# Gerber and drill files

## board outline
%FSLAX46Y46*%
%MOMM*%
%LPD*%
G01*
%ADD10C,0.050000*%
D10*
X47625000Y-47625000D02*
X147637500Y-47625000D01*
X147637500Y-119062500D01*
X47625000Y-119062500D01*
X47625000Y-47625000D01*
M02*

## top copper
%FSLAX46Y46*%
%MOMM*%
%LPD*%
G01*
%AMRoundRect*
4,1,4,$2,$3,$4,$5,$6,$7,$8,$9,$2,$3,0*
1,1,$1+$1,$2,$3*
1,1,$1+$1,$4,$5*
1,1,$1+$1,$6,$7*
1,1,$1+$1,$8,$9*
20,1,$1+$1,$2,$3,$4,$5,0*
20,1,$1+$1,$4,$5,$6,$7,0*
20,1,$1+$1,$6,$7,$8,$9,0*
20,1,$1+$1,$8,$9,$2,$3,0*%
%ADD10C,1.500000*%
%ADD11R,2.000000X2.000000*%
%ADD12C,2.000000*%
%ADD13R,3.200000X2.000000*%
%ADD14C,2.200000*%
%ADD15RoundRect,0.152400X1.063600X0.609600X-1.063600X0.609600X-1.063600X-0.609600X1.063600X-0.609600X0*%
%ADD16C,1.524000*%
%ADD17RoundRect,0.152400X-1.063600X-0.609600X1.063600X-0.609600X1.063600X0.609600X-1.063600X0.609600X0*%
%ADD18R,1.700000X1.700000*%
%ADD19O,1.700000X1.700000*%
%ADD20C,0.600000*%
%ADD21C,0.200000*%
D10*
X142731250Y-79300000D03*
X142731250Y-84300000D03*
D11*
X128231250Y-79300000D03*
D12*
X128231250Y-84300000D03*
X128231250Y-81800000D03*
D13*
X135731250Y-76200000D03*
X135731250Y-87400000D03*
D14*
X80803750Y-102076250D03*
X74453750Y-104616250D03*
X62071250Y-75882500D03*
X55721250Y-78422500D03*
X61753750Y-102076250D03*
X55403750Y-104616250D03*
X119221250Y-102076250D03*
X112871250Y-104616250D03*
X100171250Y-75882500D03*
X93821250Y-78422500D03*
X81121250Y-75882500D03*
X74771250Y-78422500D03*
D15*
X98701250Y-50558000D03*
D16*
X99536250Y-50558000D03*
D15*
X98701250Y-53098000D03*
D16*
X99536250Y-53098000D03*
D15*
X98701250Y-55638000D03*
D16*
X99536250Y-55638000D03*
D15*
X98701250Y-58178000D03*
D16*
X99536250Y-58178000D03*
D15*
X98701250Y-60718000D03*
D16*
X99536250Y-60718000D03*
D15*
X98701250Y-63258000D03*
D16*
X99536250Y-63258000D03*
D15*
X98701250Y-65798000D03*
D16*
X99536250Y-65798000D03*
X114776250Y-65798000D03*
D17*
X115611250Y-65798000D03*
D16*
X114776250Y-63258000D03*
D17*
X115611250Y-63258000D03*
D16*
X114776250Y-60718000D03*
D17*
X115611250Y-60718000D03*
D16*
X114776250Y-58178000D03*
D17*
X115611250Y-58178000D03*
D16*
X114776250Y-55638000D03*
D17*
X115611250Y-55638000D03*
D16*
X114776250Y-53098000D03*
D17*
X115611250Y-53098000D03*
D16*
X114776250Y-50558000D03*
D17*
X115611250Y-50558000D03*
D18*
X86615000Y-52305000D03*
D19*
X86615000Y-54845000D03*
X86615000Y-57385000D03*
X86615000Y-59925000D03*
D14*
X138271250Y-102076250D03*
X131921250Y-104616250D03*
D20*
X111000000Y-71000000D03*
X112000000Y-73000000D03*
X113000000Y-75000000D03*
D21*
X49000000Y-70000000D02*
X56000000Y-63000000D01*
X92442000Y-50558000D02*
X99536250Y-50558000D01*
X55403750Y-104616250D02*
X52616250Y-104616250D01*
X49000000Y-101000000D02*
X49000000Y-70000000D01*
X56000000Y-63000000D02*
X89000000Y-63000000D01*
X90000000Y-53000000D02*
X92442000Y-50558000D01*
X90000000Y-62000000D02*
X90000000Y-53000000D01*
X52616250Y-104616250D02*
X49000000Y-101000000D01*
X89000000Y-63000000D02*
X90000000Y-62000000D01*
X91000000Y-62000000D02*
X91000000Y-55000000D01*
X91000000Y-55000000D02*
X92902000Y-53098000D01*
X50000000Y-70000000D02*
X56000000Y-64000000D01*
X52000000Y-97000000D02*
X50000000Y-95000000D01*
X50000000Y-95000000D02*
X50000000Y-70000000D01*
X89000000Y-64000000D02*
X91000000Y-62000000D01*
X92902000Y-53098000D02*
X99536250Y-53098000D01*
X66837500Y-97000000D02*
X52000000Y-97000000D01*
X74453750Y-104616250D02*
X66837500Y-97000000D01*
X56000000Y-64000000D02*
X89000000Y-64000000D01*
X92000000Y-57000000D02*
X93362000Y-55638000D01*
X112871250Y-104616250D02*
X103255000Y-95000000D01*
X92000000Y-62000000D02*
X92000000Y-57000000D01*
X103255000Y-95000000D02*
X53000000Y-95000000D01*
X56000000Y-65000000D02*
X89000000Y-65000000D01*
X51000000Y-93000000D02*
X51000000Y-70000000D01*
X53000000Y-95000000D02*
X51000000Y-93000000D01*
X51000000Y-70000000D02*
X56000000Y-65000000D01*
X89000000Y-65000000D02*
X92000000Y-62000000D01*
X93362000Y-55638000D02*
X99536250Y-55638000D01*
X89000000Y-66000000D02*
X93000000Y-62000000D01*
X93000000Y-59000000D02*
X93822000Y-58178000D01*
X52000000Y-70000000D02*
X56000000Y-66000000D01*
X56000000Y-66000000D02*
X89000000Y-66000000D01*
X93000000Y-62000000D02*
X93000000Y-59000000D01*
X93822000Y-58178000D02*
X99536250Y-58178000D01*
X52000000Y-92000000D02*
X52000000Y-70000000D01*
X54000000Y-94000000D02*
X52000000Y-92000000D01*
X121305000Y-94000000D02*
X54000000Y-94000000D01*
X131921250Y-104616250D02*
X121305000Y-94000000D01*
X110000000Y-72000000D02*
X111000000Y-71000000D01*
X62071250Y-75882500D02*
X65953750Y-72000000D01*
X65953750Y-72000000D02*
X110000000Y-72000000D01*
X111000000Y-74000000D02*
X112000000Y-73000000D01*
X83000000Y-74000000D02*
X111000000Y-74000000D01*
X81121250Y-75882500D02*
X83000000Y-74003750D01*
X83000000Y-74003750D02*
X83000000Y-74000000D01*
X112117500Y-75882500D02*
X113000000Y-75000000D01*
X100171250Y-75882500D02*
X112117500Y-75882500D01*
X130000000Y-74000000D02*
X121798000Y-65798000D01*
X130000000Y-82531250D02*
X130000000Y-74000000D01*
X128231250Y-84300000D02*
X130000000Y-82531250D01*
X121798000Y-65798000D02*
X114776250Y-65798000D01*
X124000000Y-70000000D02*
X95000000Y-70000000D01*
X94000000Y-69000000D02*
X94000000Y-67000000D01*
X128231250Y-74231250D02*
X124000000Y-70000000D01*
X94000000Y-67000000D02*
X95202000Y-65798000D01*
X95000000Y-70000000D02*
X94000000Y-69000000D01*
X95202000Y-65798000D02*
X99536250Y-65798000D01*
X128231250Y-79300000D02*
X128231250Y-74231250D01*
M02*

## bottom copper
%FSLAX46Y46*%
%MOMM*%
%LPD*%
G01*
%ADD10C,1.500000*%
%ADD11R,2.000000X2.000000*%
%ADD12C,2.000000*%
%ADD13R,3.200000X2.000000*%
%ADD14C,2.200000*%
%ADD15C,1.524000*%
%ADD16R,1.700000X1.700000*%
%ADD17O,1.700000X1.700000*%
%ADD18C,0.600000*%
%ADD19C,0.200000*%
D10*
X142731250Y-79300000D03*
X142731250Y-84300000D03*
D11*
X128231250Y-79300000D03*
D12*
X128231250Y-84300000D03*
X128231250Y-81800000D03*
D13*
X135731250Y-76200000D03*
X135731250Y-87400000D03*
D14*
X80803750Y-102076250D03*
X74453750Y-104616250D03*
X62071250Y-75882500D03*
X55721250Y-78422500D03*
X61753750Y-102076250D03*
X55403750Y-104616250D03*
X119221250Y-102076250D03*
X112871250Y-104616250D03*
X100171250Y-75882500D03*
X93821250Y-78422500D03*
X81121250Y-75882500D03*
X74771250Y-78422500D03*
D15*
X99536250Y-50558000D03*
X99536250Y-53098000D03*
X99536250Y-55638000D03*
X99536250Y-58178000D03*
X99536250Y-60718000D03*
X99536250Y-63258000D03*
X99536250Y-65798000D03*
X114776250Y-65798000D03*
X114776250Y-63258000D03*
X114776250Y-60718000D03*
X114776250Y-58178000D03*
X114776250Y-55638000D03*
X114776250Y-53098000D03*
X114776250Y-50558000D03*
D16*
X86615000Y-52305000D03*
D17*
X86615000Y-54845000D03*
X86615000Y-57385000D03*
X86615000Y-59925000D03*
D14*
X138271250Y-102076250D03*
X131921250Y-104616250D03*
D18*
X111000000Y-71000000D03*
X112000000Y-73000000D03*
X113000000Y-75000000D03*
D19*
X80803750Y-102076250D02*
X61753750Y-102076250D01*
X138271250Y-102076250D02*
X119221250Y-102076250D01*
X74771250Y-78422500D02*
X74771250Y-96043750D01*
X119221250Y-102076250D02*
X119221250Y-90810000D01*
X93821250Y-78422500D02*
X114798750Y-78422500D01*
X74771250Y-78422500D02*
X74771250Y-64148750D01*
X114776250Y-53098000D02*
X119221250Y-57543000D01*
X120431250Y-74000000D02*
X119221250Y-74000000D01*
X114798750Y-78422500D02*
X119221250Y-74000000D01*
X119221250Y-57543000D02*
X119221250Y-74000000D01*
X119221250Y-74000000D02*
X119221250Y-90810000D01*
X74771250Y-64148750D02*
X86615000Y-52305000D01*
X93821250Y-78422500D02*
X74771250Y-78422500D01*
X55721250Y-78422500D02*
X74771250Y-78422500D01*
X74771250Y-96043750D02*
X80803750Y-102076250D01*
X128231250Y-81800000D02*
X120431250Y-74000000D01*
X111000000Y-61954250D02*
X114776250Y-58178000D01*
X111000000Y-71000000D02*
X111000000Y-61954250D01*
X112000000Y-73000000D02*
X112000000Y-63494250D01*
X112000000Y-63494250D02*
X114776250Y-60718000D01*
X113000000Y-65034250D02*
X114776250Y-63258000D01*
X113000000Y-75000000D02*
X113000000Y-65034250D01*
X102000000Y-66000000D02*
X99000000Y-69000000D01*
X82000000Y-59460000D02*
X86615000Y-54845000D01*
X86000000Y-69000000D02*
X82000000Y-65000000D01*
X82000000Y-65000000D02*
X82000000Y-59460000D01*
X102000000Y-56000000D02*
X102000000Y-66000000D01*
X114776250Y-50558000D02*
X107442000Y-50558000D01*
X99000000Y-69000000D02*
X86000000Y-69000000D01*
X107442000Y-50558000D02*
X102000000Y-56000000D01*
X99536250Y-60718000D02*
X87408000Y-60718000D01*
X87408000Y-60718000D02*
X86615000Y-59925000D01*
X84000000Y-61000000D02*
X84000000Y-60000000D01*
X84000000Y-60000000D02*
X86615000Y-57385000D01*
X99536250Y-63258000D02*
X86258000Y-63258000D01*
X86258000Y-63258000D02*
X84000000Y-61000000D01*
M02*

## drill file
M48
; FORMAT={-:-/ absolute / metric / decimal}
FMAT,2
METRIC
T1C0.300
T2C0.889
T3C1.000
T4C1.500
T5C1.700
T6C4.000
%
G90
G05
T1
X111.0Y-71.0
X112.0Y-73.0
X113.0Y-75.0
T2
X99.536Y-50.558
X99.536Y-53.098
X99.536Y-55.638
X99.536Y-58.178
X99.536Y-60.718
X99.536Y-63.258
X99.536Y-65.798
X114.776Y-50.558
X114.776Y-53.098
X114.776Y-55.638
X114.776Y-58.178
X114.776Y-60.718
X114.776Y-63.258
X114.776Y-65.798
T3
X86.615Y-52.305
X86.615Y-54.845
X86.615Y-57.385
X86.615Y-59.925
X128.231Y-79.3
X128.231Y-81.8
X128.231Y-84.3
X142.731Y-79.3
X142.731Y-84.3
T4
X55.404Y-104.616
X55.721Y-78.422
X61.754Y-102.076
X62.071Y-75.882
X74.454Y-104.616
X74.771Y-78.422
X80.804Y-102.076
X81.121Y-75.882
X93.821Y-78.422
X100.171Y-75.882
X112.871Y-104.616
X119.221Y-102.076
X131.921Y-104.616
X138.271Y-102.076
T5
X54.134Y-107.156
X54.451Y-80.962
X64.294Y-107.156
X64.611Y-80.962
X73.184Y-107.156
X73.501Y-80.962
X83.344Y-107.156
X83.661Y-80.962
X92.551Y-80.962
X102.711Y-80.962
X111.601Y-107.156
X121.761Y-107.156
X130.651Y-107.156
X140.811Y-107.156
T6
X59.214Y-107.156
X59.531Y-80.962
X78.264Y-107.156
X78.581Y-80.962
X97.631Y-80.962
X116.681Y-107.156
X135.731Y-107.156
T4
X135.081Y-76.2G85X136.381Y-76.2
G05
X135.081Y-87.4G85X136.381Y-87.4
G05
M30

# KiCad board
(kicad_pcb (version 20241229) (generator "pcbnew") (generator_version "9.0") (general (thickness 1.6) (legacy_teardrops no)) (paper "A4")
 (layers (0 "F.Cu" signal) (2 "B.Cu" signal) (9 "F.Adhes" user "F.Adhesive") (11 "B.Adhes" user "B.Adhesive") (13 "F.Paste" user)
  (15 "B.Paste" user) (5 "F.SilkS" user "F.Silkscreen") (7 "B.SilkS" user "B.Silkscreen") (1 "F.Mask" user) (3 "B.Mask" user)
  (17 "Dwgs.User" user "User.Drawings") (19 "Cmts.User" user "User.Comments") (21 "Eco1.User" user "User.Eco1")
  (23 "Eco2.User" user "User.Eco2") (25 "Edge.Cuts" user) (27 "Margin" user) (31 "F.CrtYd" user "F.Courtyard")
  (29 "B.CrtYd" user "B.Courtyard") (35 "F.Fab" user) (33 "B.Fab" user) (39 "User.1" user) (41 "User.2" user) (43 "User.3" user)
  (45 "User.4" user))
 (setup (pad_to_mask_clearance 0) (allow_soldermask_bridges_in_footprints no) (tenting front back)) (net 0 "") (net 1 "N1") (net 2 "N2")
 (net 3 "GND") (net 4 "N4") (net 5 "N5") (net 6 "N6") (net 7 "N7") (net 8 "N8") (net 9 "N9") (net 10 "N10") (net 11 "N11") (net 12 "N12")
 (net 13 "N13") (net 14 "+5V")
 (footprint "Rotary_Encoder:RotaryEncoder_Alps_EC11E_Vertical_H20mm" (layer "F.Cu") (at 128.23125 79.3)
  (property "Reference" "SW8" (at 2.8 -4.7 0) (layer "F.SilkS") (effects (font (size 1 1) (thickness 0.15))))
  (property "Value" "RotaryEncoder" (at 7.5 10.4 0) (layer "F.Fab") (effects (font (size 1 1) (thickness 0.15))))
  (pad "" thru_hole circle (at 14.5 0) (size 1.5 1.5) (drill 1) (layers "*.Cu" "*.Mask") (remove_unused_layers no))
  (pad "" thru_hole circle (at 14.5 5) (size 1.5 1.5) (drill 1) (layers "*.Cu" "*.Mask") (remove_unused_layers no))
  (pad "A" thru_hole rect (at 0 0) (size 2 2) (drill 1) (layers "*.Cu" "*.Mask") (remove_unused_layers no) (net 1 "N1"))
  (pad "B" thru_hole circle (at 0 5) (size 2 2) (drill 1) (layers "*.Cu" "*.Mask") (remove_unused_layers no) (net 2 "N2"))
  (pad "C" thru_hole circle (at 0 2.5) (size 2 2) (drill 1) (layers "*.Cu" "*.Mask") (remove_unused_layers no) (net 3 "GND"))
  (pad "MP" thru_hole rect (at 7.5 -3.1) (size 3.2 2) (drill oval 2.8 1.5) (layers "*.Cu" "*.Mask") (remove_unused_layers no))
  (pad "MP" thru_hole rect (at 7.5 8.1) (size 3.2 2) (drill oval 2.8 1.5) (layers "*.Cu" "*.Mask") (remove_unused_layers no)))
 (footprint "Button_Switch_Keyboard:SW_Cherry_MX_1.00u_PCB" (layer "F.Cu") (at 80.80375 102.07625)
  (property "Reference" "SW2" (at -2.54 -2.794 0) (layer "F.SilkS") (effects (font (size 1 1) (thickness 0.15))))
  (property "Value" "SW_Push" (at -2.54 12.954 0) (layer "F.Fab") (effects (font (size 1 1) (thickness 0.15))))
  (pad "" np_thru_hole circle (at -7.62 5.08) (size 1.7 1.7) (drill 1.7) (layers "*.Cu" "*.Mask"))
  (pad "" np_thru_hole circle (at -2.54 5.08) (size 4 4) (drill 4) (layers "*.Cu" "*.Mask"))
  (pad "" np_thru_hole circle (at 2.54 5.08) (size 1.7 1.7) (drill 1.7) (layers "*.Cu" "*.Mask"))
  (pad "1" thru_hole circle (at 0 0) (size 2.2 2.2) (drill 1.5) (layers "*.Cu" "*.Mask") (remove_unused_layers no) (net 3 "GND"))
  (pad "2" thru_hole circle (at -6.35 2.54) (size 2.2 2.2) (drill 1.5) (layers "*.Cu" "*.Mask") (remove_unused_layers no) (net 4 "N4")))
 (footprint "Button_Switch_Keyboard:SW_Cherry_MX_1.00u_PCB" (layer "F.Cu") (at 62.07125 75.8825)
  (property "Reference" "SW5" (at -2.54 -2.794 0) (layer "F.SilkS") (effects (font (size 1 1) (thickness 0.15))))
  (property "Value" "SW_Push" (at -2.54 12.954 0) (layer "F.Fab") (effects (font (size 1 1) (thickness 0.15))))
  (pad "" np_thru_hole circle (at -7.62 5.08) (size 1.7 1.7) (drill 1.7) (layers "*.Cu" "*.Mask"))
  (pad "" np_thru_hole circle (at -2.54 5.08) (size 4 4) (drill 4) (layers "*.Cu" "*.Mask"))
  (pad "" np_thru_hole circle (at 2.54 5.08) (size 1.7 1.7) (drill 1.7) (layers "*.Cu" "*.Mask"))
  (pad "1" thru_hole circle (at 0 0) (size 2.2 2.2) (drill 1.5) (layers "*.Cu" "*.Mask") (remove_unused_layers no) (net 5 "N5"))
  (pad "2" thru_hole circle (at -6.35 2.54) (size 2.2 2.2) (drill 1.5) (layers "*.Cu" "*.Mask") (remove_unused_layers no) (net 3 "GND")))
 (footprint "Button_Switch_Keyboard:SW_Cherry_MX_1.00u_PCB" (layer "F.Cu") (at 61.75375 102.07625)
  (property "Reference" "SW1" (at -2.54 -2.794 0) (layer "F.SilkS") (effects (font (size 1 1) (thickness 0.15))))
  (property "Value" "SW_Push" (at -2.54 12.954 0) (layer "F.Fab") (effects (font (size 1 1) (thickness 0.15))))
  (pad "" np_thru_hole circle (at -7.62 5.08) (size 1.7 1.7) (drill 1.7) (layers "*.Cu" "*.Mask"))
  (pad "" np_thru_hole circle (at -2.54 5.08) (size 4 4) (drill 4) (layers "*.Cu" "*.Mask"))
  (pad "" np_thru_hole circle (at 2.54 5.08) (size 1.7 1.7) (drill 1.7) (layers "*.Cu" "*.Mask"))
  (pad "1" thru_hole circle (at 0 0) (size 2.2 2.2) (drill 1.5) (layers "*.Cu" "*.Mask") (remove_unused_layers no) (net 3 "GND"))
  (pad "2" thru_hole circle (at -6.35 2.54) (size 2.2 2.2) (drill 1.5) (layers "*.Cu" "*.Mask") (remove_unused_layers no) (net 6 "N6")))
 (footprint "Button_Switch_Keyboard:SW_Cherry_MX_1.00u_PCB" (layer "F.Cu") (at 119.22125 102.07625)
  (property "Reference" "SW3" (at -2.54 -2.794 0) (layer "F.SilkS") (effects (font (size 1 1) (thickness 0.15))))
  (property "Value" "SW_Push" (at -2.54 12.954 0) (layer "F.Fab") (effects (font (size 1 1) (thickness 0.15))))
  (pad "" np_thru_hole circle (at -7.62 5.08) (size 1.7 1.7) (drill 1.7) (layers "*.Cu" "*.Mask"))
  (pad "" np_thru_hole circle (at -2.54 5.08) (size 4 4) (drill 4) (layers "*.Cu" "*.Mask"))
  (pad "" np_thru_hole circle (at 2.54 5.08) (size 1.7 1.7) (drill 1.7) (layers "*.Cu" "*.Mask"))
  (pad "1" thru_hole circle (at 0 0) (size 2.2 2.2) (drill 1.5) (layers "*.Cu" "*.Mask") (remove_unused_layers no) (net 3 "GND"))
  (pad "2" thru_hole circle (at -6.35 2.54) (size 2.2 2.2) (drill 1.5) (layers "*.Cu" "*.Mask") (remove_unused_layers no) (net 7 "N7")))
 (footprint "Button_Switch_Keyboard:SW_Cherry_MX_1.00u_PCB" (layer "F.Cu") (at 100.17125 75.8825)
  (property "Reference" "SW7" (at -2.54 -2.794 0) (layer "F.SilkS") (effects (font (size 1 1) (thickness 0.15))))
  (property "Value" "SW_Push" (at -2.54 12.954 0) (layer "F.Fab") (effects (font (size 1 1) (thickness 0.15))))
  (pad "" np_thru_hole circle (at -7.62 5.08) (size 1.7 1.7) (drill 1.7) (layers "*.Cu" "*.Mask"))
  (pad "" np_thru_hole circle (at -2.54 5.08) (size 4 4) (drill 4) (layers "*.Cu" "*.Mask"))
  (pad "" np_thru_hole circle (at 2.54 5.08) (size 1.7 1.7) (drill 1.7) (layers "*.Cu" "*.Mask"))
  (pad "1" thru_hole circle (at 0 0) (size 2.2 2.2) (drill 1.5) (layers "*.Cu" "*.Mask") (remove_unused_layers no) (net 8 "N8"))
  (pad "2" thru_hole circle (at -6.35 2.54) (size 2.2 2.2) (drill 1.5) (layers "*.Cu" "*.Mask") (remove_unused_layers no) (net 3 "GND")))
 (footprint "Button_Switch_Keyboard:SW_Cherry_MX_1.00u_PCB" (layer "F.Cu") (at 81.12125 75.8825)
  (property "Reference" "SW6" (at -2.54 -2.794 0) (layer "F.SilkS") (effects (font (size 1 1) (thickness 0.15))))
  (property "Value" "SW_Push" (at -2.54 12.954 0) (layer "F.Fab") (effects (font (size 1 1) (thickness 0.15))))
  (pad "" np_thru_hole circle (at -7.62 5.08) (size 1.7 1.7) (drill 1.7) (layers "*.Cu" "*.Mask"))
  (pad "" np_thru_hole circle (at -2.54 5.08) (size 4 4) (drill 4) (layers "*.Cu" "*.Mask"))
  (pad "" np_thru_hole circle (at 2.54 5.08) (size 1.7 1.7) (drill 1.7) (layers "*.Cu" "*.Mask"))
  (pad "1" thru_hole circle (at 0 0) (size 2.2 2.2) (drill 1.5) (layers "*.Cu" "*.Mask") (remove_unused_layers no) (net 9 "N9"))
  (pad "2" thru_hole circle (at -6.35 2.54) (size 2.2 2.2) (drill 1.5) (layers "*.Cu" "*.Mask") (remove_unused_layers no) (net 3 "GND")))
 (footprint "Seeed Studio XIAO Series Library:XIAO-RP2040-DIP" (layer "F.Cu") (at 107.15625 58.178)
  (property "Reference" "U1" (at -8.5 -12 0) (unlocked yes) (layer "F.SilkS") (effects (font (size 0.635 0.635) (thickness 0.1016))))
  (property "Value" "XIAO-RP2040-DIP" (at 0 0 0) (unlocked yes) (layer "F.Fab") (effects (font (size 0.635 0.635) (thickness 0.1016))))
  (pad "1" smd roundrect (at -8.455 -7.62 180) (size 2.432 1.524) (layers "F.Cu" "F.Mask") (roundrect_rratio 0.1) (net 6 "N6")
   (thermal_bridge_angle 45))
  (pad "1" thru_hole circle (at -7.62 -7.62 180) (size 1.524 1.524) (drill 0.889) (layers "*.Cu" "*.Mask") (remove_unused_layers no)
   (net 6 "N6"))
  (pad "2" smd roundrect (at -8.455 -5.08 180) (size 2.432 1.524) (layers "F.Cu" "F.Mask") (roundrect_rratio 0.1) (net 4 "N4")
   (thermal_bridge_angle 45))
  (pad "2" thru_hole circle (at -7.62 -5.08 180) (size 1.524 1.524) (drill 0.889) (layers "*.Cu" "*.Mask") (remove_unused_layers no)
   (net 4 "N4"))
  (pad "3" smd roundrect (at -8.455 -2.54 180) (size 2.432 1.524) (layers "F.Cu" "F.Mask") (roundrect_rratio 0.1) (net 7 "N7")
   (thermal_bridge_angle 45))
  (pad "3" thru_hole circle (at -7.62 -2.54 180) (size 1.524 1.524) (drill 0.889) (layers "*.Cu" "*.Mask") (remove_unused_layers no)
   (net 7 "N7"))
  (pad "4" smd roundrect (at -8.455 0 180) (size 2.432 1.524) (layers "F.Cu" "F.Mask") (roundrect_rratio 0.1) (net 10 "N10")
   (thermal_bridge_angle 45))
  (pad "4" thru_hole circle (at -7.62 0 180) (size 1.524 1.524) (drill 0.889) (layers "*.Cu" "*.Mask") (remove_unused_layers no)
   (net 10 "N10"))
  (pad "5" smd roundrect (at -8.455 2.54 180) (size 2.432 1.524) (layers "F.Cu" "F.Mask") (roundrect_rratio 0.1) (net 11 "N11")
   (thermal_bridge_angle 45))
  (pad "5" thru_hole circle (at -7.62 2.54 180) (size 1.524 1.524) (drill 0.889) (layers "*.Cu" "*.Mask") (remove_unused_layers no)
   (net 11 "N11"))
  (pad "6" smd roundrect (at -8.455 5.08 180) (size 2.432 1.524) (layers "F.Cu" "F.Mask") (roundrect_rratio 0.1) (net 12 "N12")
   (thermal_bridge_angle 45))
  (pad "6" thru_hole circle (at -7.62 5.08 180) (size 1.524 1.524) (drill 0.889) (layers "*.Cu" "*.Mask") (remove_unused_layers no)
   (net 12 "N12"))
  (pad "7" smd roundrect (at -8.455 7.62 180) (size 2.432 1.524) (layers "F.Cu" "F.Mask") (roundrect_rratio 0.1) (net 1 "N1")
   (thermal_bridge_angle 45))
  (pad "7" thru_hole circle (at -7.62 7.62 180) (size 1.524 1.524) (drill 0.889) (layers "*.Cu" "*.Mask") (remove_unused_layers no)
   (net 1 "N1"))
  (pad "8" thru_hole circle (at 7.62 7.62) (size 1.524 1.524) (drill 0.889) (layers "*.Cu" "*.Mask") (remove_unused_layers no) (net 2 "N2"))
  (pad "8" smd roundrect (at 8.455 7.62) (size 2.432 1.524) (layers "F.Cu" "F.Mask") (roundrect_rratio 0.1) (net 2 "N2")
   (thermal_bridge_angle 45))
  (pad "9" thru_hole circle (at 7.62 5.08) (size 1.524 1.524) (drill 0.889) (layers "*.Cu" "*.Mask") (remove_unused_layers no) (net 8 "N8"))
  (pad "9" smd roundrect (at 8.455 5.08) (size 2.432 1.524) (layers "F.Cu" "F.Mask") (roundrect_rratio 0.1) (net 8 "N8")
   (thermal_bridge_angle 45))
  (pad "10" thru_hole circle (at 7.62 2.54) (size 1.524 1.524) (drill 0.889) (layers "*.Cu" "*.Mask") (remove_unused_layers no) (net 9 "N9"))
  (pad "10" smd roundrect (at 8.455 2.54) (size 2.432 1.524) (layers "F.Cu" "F.Mask") (roundrect_rratio 0.1) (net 9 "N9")
   (thermal_bridge_angle 45))
  (pad "11" thru_hole circle (at 7.62 0) (size 1.524 1.524) (drill 0.889) (layers "*.Cu" "*.Mask") (remove_unused_layers no) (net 5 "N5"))
  (pad "11" smd roundrect (at 8.455 0) (size 2.432 1.524) (layers "F.Cu" "F.Mask") (roundrect_rratio 0.1) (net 5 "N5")
   (thermal_bridge_angle 45))
  (pad "12" thru_hole circle (at 7.62 -2.54) (size 1.524 1.524) (drill 0.889) (layers "*.Cu" "*.Mask") (remove_unused_layers no)
   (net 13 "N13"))
  (pad "12" smd roundrect (at 8.455 -2.54) (size 2.432 1.524) (layers "F.Cu" "F.Mask") (roundrect_rratio 0.1) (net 13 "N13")
   (thermal_bridge_angle 45))
  (pad "13" thru_hole circle (at 7.62 -5.08) (size 1.524 1.524) (drill 0.889) (layers "*.Cu" "*.Mask") (remove_unused_layers no)
   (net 3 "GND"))
  (pad "13" smd roundrect (at 8.455 -5.08) (size 2.432 1.524) (layers "F.Cu" "F.Mask") (roundrect_rratio 0.1) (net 3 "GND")
   (thermal_bridge_angle 45))
  (pad "14" thru_hole circle (at 7.62 -7.62) (size 1.524 1.524) (drill 0.889) (layers "*.Cu" "*.Mask") (remove_unused_layers no)
   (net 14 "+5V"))
  (pad "14" smd roundrect (at 8.455 -7.62) (size 2.432 1.524) (layers "F.Cu" "F.Mask") (roundrect_rratio 0.1) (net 14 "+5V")
   (thermal_bridge_angle 45)))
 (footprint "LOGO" (layer "F.Cu") (at 134 58)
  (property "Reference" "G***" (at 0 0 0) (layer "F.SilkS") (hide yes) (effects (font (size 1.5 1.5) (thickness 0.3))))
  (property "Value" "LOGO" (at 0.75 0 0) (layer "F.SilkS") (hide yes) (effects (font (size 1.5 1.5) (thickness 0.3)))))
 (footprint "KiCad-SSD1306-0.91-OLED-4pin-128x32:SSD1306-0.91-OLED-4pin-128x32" (layer "F.Cu") (at 50.115 50.115)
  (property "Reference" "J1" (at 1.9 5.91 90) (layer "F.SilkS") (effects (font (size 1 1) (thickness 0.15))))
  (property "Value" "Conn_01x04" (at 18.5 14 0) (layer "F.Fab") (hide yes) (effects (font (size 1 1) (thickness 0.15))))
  (pad "1" thru_hole rect (at 36.5 2.19) (size 1.7 1.7) (drill 1) (layers "*.Cu" "*.Mask") (remove_unused_layers no) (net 3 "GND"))
  (pad "2" thru_hole oval (at 36.5 4.73) (size 1.7 1.7) (drill 1) (layers "*.Cu" "*.Mask") (remove_unused_layers no) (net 14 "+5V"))
  (pad "3" thru_hole oval (at 36.5 7.27) (size 1.7 1.7) (drill 1) (layers "*.Cu" "*.Mask") (remove_unused_layers no) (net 12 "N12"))
  (pad "4" thru_hole oval (at 36.5 9.81) (size 1.7 1.7) (drill 1) (layers "*.Cu" "*.Mask") (remove_unused_layers no) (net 11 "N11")))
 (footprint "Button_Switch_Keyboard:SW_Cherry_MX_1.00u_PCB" (layer "F.Cu") (at 138.27125 102.07625)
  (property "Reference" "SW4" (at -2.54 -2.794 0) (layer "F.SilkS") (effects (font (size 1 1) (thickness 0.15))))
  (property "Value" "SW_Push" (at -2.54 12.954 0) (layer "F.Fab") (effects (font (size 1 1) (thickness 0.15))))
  (pad "" np_thru_hole circle (at -7.62 5.08) (size 1.7 1.7) (drill 1.7) (layers "*.Cu" "*.Mask"))
  (pad "" np_thru_hole circle (at -2.54 5.08) (size 4 4) (drill 4) (layers "*.Cu" "*.Mask"))
  (pad "" np_thru_hole circle (at 2.54 5.08) (size 1.7 1.7) (drill 1.7) (layers "*.Cu" "*.Mask"))
  (pad "1" thru_hole circle (at 0 0) (size 2.2 2.2) (drill 1.5) (layers "*.Cu" "*.Mask") (remove_unused_layers no) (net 3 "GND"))
  (pad "2" thru_hole circle (at -6.35 2.54) (size 2.2 2.2) (drill 1.5) (layers "*.Cu" "*.Mask") (remove_unused_layers no) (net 10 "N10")))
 (gr_rect (start 47.625 47.625) (end 147.6375 119.0625) (stroke (width 0.05) (type default)) (fill no) (layer "Edge.Cuts"))
 (segment (start 49 70) (end 56 63) (width 0.2) (layer "F.Cu") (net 6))
 (segment (start 92.442 50.558) (end 99.53625 50.558) (width 0.2) (layer "F.Cu") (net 6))
 (segment (start 55.40375 104.61625) (end 52.61625 104.61625) (width 0.2) (layer "F.Cu") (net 6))
 (segment (start 49 101) (end 49 70) (width 0.2) (layer "F.Cu") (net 6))
 (segment (start 56 63) (end 89 63) (width 0.2) (layer "F.Cu") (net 6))
 (segment (start 90 53) (end 92.442 50.558) (width 0.2) (layer "F.Cu") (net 6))
 (segment (start 90 62) (end 90 53) (width 0.2) (layer "F.Cu") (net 6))
 (segment (start 52.61625 104.61625) (end 49 101) (width 0.2) (layer "F.Cu") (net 6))
 (segment (start 89 63) (end 90 62) (width 0.2) (layer "F.Cu") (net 6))
 (segment (start 80.80375 102.07625) (end 61.75375 102.07625) (width 0.2) (layer "B.Cu") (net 3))
 (segment (start 138.27125 102.07625) (end 119.22125 102.07625) (width 0.2) (layer "B.Cu") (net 3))
 (segment (start 74.77125 78.4225) (end 74.77125 96.04375) (width 0.2) (layer "B.Cu") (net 3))
 (segment (start 119.22125 102.07625) (end 119.22125 90.81) (width 0.2) (layer "B.Cu") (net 3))
 (segment (start 93.82125 78.4225) (end 114.79875 78.4225) (width 0.2) (layer "B.Cu") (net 3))
 (segment (start 74.77125 78.4225) (end 74.77125 64.14875) (width 0.2) (layer "B.Cu") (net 3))
 (segment (start 114.77625 53.098) (end 119.22125 57.543) (width 0.2) (layer "B.Cu") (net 3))
 (segment (start 120.43125 74) (end 119.22125 74) (width 0.2) (layer "B.Cu") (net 3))
 (segment (start 114.79875 78.4225) (end 119.22125 74) (width 0.2) (layer "B.Cu") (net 3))
 (segment (start 119.22125 57.543) (end 119.22125 74) (width 0.2) (layer "B.Cu") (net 3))
 (segment (start 119.22125 74) (end 119.22125 90.81) (width 0.2) (layer "B.Cu") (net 3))
 (segment (start 74.77125 64.14875) (end 86.615 52.305) (width 0.2) (layer "B.Cu") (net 3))
 (segment (start 93.82125 78.4225) (end 74.77125 78.4225) (width 0.2) (layer "B.Cu") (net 3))
 (segment (start 55.72125 78.4225) (end 74.77125 78.4225) (width 0.2) (layer "B.Cu") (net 3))
 (segment (start 74.77125 96.04375) (end 80.80375 102.07625) (width 0.2) (layer "B.Cu") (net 3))
 (segment (start 128.23125 81.8) (end 120.43125 74) (width 0.2) (layer "B.Cu") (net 3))
 (segment (start 91 62) (end 91 55) (width 0.2) (layer "F.Cu") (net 4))
 (segment (start 91 55) (end 92.902 53.098) (width 0.2) (layer "F.Cu") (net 4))
 (segment (start 50 70) (end 56 64) (width 0.2) (layer "F.Cu") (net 4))
 (segment (start 52 97) (end 50 95) (width 0.2) (layer "F.Cu") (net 4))
 (segment (start 50 95) (end 50 70) (width 0.2) (layer "F.Cu") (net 4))
 (segment (start 89 64) (end 91 62) (width 0.2) (layer "F.Cu") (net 4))
 (segment (start 92.902 53.098) (end 99.53625 53.098) (width 0.2) (layer "F.Cu") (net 4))
 (segment (start 66.8375 97) (end 52 97) (width 0.2) (layer "F.Cu") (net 4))
 (segment (start 74.45375 104.61625) (end 66.8375 97) (width 0.2) (layer "F.Cu") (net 4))
 (segment (start 56 64) (end 89 64) (width 0.2) (layer "F.Cu") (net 4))
 (segment (start 92 57) (end 93.362 55.638) (width 0.2) (layer "F.Cu") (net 7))
 (segment (start 112.87125 104.61625) (end 103.255 95) (width 0.2) (layer "F.Cu") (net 7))
 (segment (start 92 62) (end 92 57) (width 0.2) (layer "F.Cu") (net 7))
 (segment (start 103.255 95) (end 53 95) (width 0.2) (layer "F.Cu") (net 7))
 (segment (start 56 65) (end 89 65) (width 0.2) (layer "F.Cu") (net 7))
 (segment (start 51 93) (end 51 70) (width 0.2) (layer "F.Cu") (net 7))
 (segment (start 53 95) (end 51 93) (width 0.2) (layer "F.Cu") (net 7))
 (segment (start 51 70) (end 56 65) (width 0.2) (layer "F.Cu") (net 7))
 (segment (start 89 65) (end 92 62) (width 0.2) (layer "F.Cu") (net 7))
 (segment (start 93.362 55.638) (end 99.53625 55.638) (width 0.2) (layer "F.Cu") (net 7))
 (segment (start 89 66) (end 93 62) (width 0.2) (layer "F.Cu") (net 10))
 (segment (start 93 59) (end 93.822 58.178) (width 0.2) (layer "F.Cu") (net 10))
 (segment (start 52 70) (end 56 66) (width 0.2) (layer "F.Cu") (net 10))
 (segment (start 56 66) (end 89 66) (width 0.2) (layer "F.Cu") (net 10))
 (segment (start 93 62) (end 93 59) (width 0.2) (layer "F.Cu") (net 10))
 (segment (start 93.822 58.178) (end 99.53625 58.178) (width 0.2) (layer "F.Cu") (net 10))
 (segment (start 52 92) (end 52 70) (width 0.2) (layer "F.Cu") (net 10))
 (segment (start 54 94) (end 52 92) (width 0.2) (layer "F.Cu") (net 10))
 (segment (start 121.305 94) (end 54 94) (width 0.2) (layer "F.Cu") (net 10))
 (segment (start 131.92125 104.61625) (end 121.305 94) (width 0.2) (layer "F.Cu") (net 10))
 (segment (start 110 72) (end 111 71) (width 0.2) (layer "F.Cu") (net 5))
 (segment (start 62.07125 75.8825) (end 65.95375 72) (width 0.2) (layer "F.Cu") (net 5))
 (segment (start 65.95375 72) (end 110 72) (width 0.2) (layer "F.Cu") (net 5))
 (via (at 111 71) (size 0.6) (drill 0.3) (layers "F.Cu" "B.Cu") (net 5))
 (segment (start 111 61.95425) (end 114.77625 58.178) (width 0.2) (layer "B.Cu") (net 5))
 (segment (start 111 71) (end 111 61.95425) (width 0.2) (layer "B.Cu") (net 5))
 (segment (start 111 74) (end 112 73) (width 0.2) (layer "F.Cu") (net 9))
 (segment (start 83 74) (end 111 74) (width 0.2) (layer "F.Cu") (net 9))
 (segment (start 81.12125 75.8825) (end 83 74.00375) (width 0.2) (layer "F.Cu") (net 9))
 (segment (start 83 74.00375) (end 83 74) (width 0.2) (layer "F.Cu") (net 9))
 (via (at 112 73) (size 0.6) (drill 0.3) (layers "F.Cu" "B.Cu") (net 9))
 (segment (start 112 73) (end 112 63.49425) (width 0.2) (layer "B.Cu") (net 9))
 (segment (start 112 63.49425) (end 114.77625 60.718) (width 0.2) (layer "B.Cu") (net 9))
 (segment (start 112.1175 75.8825) (end 113 75) (width 0.2) (layer "F.Cu") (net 8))
 (segment (start 100.17125 75.8825) (end 112.1175 75.8825) (width 0.2) (layer "F.Cu") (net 8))
 (via (at 113 75) (size 0.6) (drill 0.3) (layers "F.Cu" "B.Cu") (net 8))
 (segment (start 113 65.03425) (end 114.77625 63.258) (width 0.2) (layer "B.Cu") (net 8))
 (segment (start 113 75) (end 113 65.03425) (width 0.2) (layer "B.Cu") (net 8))
 (segment (start 130 74) (end 121.798 65.798) (width 0.2) (layer "F.Cu") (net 2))
 (segment (start 130 82.53125) (end 130 74) (width 0.2) (layer "F.Cu") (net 2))
 (segment (start 128.23125 84.3) (end 130 82.53125) (width 0.2) (layer "F.Cu") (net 2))
 (segment (start 121.798 65.798) (end 114.77625 65.798) (width 0.2) (layer "F.Cu") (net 2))
 (segment (start 124 70) (end 95 70) (width 0.2) (layer "F.Cu") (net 1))
 (segment (start 94 69) (end 94 67) (width 0.2) (layer "F.Cu") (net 1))
 (segment (start 128.23125 74.23125) (end 124 70) (width 0.2) (layer "F.Cu") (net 1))
 (segment (start 94 67) (end 95.202 65.798) (width 0.2) (layer "F.Cu") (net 1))
 (segment (start 95 70) (end 94 69) (width 0.2) (layer "F.Cu") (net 1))
 (segment (start 95.202 65.798) (end 99.53625 65.798) (width 0.2) (layer "F.Cu") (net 1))
 (segment (start 128.23125 79.3) (end 128.23125 74.23125) (width 0.2) (layer "F.Cu") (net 1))
 (segment (start 102 66) (end 99 69) (width 0.2) (layer "B.Cu") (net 14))
 (segment (start 82 59.46) (end 86.615 54.845) (width 0.2) (layer "B.Cu") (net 14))
 (segment (start 86 69) (end 82 65) (width 0.2) (layer "B.Cu") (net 14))
 (segment (start 82 65) (end 82 59.46) (width 0.2) (layer "B.Cu") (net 14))
 (segment (start 102 56) (end 102 66) (width 0.2) (layer "B.Cu") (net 14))
 (segment (start 114.77625 50.558) (end 107.442 50.558) (width 0.2) (layer "B.Cu") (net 14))
 (segment (start 99 69) (end 86 69) (width 0.2) (layer "B.Cu") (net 14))
 (segment (start 107.442 50.558) (end 102 56) (width 0.2) (layer "B.Cu") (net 14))
 (segment (start 99.53625 60.718) (end 87.408 60.718) (width 0.2) (layer "B.Cu") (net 11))
 (segment (start 87.408 60.718) (end 86.615 59.925) (width 0.2) (layer "B.Cu") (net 11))
 (segment (start 84 61) (end 84 60) (width 0.2) (layer "B.Cu") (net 12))
 (segment (start 84 60) (end 86.615 57.385) (width 0.2) (layer "B.Cu") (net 12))
 (segment (start 99.53625 63.258) (end 86.258 63.258) (width 0.2) (layer "B.Cu") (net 12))
 (segment (start 86.258 63.258) (end 84 61) (width 0.2) (layer "B.Cu") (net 12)))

